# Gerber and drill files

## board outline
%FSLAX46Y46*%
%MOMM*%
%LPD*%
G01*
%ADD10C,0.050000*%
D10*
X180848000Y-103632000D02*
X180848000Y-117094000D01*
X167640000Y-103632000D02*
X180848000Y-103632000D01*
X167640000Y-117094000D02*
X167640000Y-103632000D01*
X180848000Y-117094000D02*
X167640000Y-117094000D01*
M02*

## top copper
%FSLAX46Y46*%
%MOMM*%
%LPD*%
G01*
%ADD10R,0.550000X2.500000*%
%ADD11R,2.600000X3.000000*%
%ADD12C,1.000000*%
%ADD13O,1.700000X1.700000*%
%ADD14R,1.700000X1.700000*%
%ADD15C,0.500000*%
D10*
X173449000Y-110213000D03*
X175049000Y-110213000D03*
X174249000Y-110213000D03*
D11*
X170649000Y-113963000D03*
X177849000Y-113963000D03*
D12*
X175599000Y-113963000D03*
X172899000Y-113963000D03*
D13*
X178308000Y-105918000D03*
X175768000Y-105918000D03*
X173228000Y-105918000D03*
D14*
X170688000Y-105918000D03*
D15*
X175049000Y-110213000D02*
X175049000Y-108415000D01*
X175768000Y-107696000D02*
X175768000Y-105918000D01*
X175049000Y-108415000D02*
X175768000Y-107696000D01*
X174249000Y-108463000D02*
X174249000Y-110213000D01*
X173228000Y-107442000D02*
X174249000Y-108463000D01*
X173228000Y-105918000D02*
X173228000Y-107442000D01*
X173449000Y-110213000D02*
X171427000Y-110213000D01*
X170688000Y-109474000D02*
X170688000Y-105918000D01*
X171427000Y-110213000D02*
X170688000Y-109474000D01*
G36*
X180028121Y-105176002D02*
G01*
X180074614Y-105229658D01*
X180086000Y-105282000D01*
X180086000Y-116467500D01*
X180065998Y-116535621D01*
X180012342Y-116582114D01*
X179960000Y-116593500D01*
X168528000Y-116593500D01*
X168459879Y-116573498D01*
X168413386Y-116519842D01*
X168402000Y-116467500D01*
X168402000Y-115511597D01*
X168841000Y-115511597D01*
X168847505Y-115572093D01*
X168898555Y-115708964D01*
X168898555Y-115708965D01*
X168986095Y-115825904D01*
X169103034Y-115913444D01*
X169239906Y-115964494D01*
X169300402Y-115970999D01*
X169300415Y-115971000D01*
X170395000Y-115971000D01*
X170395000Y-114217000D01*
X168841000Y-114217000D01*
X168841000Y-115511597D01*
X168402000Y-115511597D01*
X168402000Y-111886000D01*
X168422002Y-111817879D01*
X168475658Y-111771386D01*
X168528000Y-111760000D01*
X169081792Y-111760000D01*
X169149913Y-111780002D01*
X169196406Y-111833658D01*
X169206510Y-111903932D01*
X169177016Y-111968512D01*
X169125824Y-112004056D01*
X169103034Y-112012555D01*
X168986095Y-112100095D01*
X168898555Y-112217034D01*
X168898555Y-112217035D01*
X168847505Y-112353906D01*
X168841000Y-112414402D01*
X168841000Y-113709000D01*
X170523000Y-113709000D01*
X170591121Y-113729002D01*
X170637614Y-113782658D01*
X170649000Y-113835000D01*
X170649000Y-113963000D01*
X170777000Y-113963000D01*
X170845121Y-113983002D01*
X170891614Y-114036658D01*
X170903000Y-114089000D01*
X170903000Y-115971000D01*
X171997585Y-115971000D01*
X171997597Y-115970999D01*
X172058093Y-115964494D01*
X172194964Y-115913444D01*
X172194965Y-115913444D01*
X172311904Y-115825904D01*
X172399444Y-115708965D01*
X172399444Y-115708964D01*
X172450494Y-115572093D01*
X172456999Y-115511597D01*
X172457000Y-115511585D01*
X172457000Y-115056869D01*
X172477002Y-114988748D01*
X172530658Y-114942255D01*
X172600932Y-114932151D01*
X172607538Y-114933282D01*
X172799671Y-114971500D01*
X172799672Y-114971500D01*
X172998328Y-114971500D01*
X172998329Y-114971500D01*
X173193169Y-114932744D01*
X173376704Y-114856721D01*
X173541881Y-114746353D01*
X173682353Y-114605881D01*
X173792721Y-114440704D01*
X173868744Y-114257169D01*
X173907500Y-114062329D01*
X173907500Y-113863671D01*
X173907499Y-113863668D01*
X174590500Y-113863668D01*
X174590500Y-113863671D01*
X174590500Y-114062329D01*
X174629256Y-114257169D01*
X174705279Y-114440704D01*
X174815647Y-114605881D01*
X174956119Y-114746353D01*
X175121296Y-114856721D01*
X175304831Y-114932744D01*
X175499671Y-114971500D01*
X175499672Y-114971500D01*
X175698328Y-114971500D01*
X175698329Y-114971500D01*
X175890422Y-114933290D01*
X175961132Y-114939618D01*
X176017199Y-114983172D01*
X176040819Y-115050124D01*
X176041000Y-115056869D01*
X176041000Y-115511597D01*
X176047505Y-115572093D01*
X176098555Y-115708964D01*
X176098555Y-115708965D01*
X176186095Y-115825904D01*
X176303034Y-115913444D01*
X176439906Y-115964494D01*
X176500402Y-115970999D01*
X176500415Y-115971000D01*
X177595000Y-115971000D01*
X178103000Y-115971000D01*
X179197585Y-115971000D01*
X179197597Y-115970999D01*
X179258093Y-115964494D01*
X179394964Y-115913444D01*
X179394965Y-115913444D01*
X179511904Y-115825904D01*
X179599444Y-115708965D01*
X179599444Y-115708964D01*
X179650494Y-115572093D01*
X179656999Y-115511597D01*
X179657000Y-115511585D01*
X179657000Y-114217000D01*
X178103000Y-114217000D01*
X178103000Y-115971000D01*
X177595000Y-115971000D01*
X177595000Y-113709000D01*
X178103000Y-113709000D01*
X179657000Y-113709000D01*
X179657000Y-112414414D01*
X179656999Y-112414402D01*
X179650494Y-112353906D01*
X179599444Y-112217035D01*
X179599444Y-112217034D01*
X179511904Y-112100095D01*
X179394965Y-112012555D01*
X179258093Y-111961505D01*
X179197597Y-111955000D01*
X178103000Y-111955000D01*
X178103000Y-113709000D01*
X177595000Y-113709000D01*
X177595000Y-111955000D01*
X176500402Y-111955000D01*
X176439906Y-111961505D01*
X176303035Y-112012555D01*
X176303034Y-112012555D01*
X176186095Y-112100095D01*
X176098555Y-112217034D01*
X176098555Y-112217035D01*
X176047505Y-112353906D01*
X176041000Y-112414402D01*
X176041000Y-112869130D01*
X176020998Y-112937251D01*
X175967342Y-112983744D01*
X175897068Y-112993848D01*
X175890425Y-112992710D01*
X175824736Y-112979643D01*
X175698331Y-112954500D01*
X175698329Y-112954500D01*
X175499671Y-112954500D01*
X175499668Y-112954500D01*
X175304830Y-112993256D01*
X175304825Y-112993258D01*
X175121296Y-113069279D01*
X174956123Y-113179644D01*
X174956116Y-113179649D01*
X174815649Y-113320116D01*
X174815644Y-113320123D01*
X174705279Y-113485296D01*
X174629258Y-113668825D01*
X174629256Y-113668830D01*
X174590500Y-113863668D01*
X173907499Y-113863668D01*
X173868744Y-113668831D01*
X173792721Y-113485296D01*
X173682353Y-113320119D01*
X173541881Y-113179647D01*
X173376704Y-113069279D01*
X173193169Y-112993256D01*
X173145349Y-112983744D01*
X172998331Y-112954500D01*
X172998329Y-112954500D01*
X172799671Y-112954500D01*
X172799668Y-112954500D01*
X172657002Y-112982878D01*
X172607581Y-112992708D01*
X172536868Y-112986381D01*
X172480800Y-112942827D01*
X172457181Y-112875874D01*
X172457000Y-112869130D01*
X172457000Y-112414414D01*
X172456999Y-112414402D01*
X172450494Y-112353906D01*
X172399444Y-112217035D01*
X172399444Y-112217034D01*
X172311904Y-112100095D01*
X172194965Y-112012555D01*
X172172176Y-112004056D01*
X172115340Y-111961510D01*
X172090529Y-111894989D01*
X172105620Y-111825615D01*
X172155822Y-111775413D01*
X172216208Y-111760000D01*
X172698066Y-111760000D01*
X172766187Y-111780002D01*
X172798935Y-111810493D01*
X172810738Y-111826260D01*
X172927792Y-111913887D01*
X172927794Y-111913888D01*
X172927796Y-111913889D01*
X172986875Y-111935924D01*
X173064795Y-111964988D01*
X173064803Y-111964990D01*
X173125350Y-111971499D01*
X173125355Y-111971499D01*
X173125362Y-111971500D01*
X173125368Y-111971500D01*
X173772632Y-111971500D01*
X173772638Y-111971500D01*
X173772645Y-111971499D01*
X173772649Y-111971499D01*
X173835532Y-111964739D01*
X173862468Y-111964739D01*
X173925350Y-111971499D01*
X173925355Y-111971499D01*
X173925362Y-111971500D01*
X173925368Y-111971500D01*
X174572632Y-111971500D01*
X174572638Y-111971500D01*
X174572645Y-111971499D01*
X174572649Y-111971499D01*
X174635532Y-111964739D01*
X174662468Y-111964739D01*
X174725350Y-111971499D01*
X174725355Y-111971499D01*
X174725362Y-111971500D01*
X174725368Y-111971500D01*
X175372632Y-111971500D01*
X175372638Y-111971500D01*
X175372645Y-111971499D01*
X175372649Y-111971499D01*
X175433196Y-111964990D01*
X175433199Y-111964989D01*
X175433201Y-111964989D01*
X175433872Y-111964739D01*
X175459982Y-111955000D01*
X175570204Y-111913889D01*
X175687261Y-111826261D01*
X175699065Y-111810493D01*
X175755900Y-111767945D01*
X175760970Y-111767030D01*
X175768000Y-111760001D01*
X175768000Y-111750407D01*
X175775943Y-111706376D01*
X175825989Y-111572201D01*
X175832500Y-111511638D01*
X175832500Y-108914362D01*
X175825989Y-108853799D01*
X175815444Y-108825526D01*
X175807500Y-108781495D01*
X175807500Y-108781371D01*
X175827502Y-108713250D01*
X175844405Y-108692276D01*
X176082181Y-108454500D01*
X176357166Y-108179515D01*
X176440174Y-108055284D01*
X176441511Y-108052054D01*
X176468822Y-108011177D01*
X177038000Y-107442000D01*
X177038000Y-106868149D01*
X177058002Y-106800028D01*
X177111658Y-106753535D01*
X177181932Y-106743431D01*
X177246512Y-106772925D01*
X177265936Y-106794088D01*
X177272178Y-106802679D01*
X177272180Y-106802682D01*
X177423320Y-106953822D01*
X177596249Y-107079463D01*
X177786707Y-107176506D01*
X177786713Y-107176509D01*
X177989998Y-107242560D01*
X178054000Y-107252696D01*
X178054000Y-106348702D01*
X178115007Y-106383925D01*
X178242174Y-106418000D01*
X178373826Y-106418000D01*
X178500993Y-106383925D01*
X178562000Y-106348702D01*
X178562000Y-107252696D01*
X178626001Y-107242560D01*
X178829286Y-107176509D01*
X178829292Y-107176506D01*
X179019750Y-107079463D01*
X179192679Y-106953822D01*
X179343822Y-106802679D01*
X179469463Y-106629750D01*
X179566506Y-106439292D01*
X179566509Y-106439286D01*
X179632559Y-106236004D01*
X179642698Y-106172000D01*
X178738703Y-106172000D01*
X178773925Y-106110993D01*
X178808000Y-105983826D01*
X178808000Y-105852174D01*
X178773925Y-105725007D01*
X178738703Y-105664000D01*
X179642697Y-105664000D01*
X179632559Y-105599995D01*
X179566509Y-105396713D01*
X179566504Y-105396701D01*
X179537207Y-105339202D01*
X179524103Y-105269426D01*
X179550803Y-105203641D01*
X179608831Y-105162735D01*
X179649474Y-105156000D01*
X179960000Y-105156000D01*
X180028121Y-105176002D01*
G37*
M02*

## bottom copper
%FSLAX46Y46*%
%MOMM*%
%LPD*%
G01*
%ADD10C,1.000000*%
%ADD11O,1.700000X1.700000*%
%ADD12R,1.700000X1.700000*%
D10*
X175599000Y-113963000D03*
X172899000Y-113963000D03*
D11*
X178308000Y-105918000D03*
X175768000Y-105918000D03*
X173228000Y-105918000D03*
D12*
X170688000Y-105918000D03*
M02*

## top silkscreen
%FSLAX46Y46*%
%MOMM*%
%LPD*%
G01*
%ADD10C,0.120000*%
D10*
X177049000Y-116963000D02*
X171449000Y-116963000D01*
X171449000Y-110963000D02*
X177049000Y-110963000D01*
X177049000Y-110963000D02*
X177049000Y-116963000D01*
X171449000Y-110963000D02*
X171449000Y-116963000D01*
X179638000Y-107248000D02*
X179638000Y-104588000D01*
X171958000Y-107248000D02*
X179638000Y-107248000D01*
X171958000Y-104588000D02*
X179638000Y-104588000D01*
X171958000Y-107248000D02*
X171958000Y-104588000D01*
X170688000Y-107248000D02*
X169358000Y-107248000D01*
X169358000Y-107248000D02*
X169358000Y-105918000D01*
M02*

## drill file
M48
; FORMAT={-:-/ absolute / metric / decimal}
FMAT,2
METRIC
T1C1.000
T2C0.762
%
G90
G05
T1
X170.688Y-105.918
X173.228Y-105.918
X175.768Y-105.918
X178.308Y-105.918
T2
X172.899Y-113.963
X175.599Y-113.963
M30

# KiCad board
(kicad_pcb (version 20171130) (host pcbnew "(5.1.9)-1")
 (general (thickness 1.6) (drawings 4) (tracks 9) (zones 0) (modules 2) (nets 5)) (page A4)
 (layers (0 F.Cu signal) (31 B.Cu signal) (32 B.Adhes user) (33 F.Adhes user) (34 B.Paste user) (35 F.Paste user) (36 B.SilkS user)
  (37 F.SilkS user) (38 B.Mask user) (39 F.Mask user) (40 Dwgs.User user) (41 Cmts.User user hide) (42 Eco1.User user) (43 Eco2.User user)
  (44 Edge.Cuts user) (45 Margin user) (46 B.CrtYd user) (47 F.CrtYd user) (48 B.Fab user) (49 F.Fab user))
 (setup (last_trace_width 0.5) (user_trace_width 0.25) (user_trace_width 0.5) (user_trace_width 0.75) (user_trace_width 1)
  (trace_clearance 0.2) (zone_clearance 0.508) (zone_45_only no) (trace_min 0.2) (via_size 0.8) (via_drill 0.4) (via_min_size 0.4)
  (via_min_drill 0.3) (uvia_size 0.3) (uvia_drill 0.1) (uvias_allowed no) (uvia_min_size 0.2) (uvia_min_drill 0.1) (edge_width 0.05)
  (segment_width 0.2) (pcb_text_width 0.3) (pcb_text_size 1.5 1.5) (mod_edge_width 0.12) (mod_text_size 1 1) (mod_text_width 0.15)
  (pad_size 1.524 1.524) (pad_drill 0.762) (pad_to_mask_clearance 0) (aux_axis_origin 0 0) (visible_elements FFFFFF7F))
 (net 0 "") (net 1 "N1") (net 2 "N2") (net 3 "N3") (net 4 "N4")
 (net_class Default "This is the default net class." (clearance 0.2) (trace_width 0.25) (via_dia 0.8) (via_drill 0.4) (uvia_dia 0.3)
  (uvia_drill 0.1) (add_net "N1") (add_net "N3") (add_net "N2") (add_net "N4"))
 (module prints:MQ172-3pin (layer F.Cu) (at 174.249 113.963)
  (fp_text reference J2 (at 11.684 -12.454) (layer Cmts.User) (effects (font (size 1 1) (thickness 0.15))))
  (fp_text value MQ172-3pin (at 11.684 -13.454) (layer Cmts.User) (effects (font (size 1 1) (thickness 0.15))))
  (fp_line (start 2.8 3) (end -2.8 3) (layer F.SilkS) (width 0.12))
  (fp_line (start -2.8 -3) (end 2.8 -3) (layer F.SilkS) (width 0.12))
  (fp_line (start 2.8 -3) (end 2.8 3) (layer F.SilkS) (width 0.12))
  (fp_line (start -2.8 -3) (end -2.8 3) (layer F.SilkS) (width 0.12))
  (pad 1 smd rect (at -0.8 -3.75) (size 0.55 2.5) (layers F.Cu F.Paste F.Mask) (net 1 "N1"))
  (pad 3 smd rect (at 0.8 -3.75) (size 0.55 2.5) (layers F.Cu F.Paste F.Mask) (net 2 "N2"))
  (pad 2 smd rect (at 0 -3.75) (size 0.55 2.5) (layers F.Cu F.Paste F.Mask) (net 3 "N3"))
  (pad 0 smd rect (at -3.6 0) (size 2.6 3) (layers F.Cu F.Paste F.Mask) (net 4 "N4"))
  (pad 0 smd rect (at 3.6 0) (size 2.6 3) (layers F.Cu F.Paste F.Mask) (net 4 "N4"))
  (pad "" np_thru_hole circle (at 1.35 0) (size 1 1) (drill 0.762) (layers *.Cu *.Mask))
  (pad "" np_thru_hole circle (at -1.35 0) (size 1 1) (drill 0.762) (layers *.Cu *.Mask)))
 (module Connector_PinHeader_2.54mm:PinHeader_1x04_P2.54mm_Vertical (layer F.Cu) (at 170.688 105.918 90)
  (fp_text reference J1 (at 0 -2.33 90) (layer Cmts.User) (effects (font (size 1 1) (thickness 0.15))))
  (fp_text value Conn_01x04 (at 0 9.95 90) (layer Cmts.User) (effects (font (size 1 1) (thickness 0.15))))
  (fp_line (start -1.33 8.95) (end 1.33 8.95) (layer F.SilkS) (width 0.12))
  (fp_line (start -1.33 1.27) (end -1.33 8.95) (layer F.SilkS) (width 0.12))
  (fp_line (start 1.33 1.27) (end 1.33 8.95) (layer F.SilkS) (width 0.12))
  (fp_line (start -1.33 1.27) (end 1.33 1.27) (layer F.SilkS) (width 0.12))
  (fp_line (start -1.33 0) (end -1.33 -1.33) (layer F.SilkS) (width 0.12))
  (fp_line (start -1.33 -1.33) (end 0 -1.33) (layer F.SilkS) (width 0.12))
  (pad 4 thru_hole oval (at 0 7.62 90) (size 1.7 1.7) (drill 1) (layers *.Cu *.Mask) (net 4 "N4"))
  (pad 3 thru_hole oval (at 0 5.08 90) (size 1.7 1.7) (drill 1) (layers *.Cu *.Mask) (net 2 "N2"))
  (pad 2 thru_hole oval (at 0 2.54 90) (size 1.7 1.7) (drill 1) (layers *.Cu *.Mask) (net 3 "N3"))
  (pad 1 thru_hole rect (at 0 0 90) (size 1.7 1.7) (drill 1) (layers *.Cu *.Mask) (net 1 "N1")))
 (gr_line (start 180.848 103.632) (end 180.848 117.094) (layer Edge.Cuts) (width 0.05))
 (gr_line (start 167.64 103.632) (end 180.848 103.632) (layer Edge.Cuts) (width 0.05))
 (gr_line (start 167.64 117.094) (end 167.64 103.632) (layer Edge.Cuts) (width 0.05))
 (gr_line (start 180.848 117.094) (end 167.64 117.094) (layer Edge.Cuts) (width 0.05))
 (segment (start 175.049 110.213) (end 175.049 108.415) (width 0.5) (layer F.Cu) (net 2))
 (segment (start 175.768 107.696) (end 175.768 105.918) (width 0.5) (layer F.Cu) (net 2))
 (segment (start 175.049 108.415) (end 175.768 107.696) (width 0.5) (layer F.Cu) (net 2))
 (segment (start 174.249 108.463) (end 174.249 110.213) (width 0.5) (layer F.Cu) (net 3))
 (segment (start 173.228 107.442) (end 174.249 108.463) (width 0.5) (layer F.Cu) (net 3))
 (segment (start 173.228 105.918) (end 173.228 107.442) (width 0.5) (layer F.Cu) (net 3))
 (segment (start 173.449 110.213) (end 171.427 110.213) (width 0.5) (layer F.Cu) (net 1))
 (segment (start 170.688 109.474) (end 170.688 105.918) (width 0.5) (layer F.Cu) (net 1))
 (segment (start 171.427 110.213) (end 170.688 109.474) (width 0.5) (layer F.Cu) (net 1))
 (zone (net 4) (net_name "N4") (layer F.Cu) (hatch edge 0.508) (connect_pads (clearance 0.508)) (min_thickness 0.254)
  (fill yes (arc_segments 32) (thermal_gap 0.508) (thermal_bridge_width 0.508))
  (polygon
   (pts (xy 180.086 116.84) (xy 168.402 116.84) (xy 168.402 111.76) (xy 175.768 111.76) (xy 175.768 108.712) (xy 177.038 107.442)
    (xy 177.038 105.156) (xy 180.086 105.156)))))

